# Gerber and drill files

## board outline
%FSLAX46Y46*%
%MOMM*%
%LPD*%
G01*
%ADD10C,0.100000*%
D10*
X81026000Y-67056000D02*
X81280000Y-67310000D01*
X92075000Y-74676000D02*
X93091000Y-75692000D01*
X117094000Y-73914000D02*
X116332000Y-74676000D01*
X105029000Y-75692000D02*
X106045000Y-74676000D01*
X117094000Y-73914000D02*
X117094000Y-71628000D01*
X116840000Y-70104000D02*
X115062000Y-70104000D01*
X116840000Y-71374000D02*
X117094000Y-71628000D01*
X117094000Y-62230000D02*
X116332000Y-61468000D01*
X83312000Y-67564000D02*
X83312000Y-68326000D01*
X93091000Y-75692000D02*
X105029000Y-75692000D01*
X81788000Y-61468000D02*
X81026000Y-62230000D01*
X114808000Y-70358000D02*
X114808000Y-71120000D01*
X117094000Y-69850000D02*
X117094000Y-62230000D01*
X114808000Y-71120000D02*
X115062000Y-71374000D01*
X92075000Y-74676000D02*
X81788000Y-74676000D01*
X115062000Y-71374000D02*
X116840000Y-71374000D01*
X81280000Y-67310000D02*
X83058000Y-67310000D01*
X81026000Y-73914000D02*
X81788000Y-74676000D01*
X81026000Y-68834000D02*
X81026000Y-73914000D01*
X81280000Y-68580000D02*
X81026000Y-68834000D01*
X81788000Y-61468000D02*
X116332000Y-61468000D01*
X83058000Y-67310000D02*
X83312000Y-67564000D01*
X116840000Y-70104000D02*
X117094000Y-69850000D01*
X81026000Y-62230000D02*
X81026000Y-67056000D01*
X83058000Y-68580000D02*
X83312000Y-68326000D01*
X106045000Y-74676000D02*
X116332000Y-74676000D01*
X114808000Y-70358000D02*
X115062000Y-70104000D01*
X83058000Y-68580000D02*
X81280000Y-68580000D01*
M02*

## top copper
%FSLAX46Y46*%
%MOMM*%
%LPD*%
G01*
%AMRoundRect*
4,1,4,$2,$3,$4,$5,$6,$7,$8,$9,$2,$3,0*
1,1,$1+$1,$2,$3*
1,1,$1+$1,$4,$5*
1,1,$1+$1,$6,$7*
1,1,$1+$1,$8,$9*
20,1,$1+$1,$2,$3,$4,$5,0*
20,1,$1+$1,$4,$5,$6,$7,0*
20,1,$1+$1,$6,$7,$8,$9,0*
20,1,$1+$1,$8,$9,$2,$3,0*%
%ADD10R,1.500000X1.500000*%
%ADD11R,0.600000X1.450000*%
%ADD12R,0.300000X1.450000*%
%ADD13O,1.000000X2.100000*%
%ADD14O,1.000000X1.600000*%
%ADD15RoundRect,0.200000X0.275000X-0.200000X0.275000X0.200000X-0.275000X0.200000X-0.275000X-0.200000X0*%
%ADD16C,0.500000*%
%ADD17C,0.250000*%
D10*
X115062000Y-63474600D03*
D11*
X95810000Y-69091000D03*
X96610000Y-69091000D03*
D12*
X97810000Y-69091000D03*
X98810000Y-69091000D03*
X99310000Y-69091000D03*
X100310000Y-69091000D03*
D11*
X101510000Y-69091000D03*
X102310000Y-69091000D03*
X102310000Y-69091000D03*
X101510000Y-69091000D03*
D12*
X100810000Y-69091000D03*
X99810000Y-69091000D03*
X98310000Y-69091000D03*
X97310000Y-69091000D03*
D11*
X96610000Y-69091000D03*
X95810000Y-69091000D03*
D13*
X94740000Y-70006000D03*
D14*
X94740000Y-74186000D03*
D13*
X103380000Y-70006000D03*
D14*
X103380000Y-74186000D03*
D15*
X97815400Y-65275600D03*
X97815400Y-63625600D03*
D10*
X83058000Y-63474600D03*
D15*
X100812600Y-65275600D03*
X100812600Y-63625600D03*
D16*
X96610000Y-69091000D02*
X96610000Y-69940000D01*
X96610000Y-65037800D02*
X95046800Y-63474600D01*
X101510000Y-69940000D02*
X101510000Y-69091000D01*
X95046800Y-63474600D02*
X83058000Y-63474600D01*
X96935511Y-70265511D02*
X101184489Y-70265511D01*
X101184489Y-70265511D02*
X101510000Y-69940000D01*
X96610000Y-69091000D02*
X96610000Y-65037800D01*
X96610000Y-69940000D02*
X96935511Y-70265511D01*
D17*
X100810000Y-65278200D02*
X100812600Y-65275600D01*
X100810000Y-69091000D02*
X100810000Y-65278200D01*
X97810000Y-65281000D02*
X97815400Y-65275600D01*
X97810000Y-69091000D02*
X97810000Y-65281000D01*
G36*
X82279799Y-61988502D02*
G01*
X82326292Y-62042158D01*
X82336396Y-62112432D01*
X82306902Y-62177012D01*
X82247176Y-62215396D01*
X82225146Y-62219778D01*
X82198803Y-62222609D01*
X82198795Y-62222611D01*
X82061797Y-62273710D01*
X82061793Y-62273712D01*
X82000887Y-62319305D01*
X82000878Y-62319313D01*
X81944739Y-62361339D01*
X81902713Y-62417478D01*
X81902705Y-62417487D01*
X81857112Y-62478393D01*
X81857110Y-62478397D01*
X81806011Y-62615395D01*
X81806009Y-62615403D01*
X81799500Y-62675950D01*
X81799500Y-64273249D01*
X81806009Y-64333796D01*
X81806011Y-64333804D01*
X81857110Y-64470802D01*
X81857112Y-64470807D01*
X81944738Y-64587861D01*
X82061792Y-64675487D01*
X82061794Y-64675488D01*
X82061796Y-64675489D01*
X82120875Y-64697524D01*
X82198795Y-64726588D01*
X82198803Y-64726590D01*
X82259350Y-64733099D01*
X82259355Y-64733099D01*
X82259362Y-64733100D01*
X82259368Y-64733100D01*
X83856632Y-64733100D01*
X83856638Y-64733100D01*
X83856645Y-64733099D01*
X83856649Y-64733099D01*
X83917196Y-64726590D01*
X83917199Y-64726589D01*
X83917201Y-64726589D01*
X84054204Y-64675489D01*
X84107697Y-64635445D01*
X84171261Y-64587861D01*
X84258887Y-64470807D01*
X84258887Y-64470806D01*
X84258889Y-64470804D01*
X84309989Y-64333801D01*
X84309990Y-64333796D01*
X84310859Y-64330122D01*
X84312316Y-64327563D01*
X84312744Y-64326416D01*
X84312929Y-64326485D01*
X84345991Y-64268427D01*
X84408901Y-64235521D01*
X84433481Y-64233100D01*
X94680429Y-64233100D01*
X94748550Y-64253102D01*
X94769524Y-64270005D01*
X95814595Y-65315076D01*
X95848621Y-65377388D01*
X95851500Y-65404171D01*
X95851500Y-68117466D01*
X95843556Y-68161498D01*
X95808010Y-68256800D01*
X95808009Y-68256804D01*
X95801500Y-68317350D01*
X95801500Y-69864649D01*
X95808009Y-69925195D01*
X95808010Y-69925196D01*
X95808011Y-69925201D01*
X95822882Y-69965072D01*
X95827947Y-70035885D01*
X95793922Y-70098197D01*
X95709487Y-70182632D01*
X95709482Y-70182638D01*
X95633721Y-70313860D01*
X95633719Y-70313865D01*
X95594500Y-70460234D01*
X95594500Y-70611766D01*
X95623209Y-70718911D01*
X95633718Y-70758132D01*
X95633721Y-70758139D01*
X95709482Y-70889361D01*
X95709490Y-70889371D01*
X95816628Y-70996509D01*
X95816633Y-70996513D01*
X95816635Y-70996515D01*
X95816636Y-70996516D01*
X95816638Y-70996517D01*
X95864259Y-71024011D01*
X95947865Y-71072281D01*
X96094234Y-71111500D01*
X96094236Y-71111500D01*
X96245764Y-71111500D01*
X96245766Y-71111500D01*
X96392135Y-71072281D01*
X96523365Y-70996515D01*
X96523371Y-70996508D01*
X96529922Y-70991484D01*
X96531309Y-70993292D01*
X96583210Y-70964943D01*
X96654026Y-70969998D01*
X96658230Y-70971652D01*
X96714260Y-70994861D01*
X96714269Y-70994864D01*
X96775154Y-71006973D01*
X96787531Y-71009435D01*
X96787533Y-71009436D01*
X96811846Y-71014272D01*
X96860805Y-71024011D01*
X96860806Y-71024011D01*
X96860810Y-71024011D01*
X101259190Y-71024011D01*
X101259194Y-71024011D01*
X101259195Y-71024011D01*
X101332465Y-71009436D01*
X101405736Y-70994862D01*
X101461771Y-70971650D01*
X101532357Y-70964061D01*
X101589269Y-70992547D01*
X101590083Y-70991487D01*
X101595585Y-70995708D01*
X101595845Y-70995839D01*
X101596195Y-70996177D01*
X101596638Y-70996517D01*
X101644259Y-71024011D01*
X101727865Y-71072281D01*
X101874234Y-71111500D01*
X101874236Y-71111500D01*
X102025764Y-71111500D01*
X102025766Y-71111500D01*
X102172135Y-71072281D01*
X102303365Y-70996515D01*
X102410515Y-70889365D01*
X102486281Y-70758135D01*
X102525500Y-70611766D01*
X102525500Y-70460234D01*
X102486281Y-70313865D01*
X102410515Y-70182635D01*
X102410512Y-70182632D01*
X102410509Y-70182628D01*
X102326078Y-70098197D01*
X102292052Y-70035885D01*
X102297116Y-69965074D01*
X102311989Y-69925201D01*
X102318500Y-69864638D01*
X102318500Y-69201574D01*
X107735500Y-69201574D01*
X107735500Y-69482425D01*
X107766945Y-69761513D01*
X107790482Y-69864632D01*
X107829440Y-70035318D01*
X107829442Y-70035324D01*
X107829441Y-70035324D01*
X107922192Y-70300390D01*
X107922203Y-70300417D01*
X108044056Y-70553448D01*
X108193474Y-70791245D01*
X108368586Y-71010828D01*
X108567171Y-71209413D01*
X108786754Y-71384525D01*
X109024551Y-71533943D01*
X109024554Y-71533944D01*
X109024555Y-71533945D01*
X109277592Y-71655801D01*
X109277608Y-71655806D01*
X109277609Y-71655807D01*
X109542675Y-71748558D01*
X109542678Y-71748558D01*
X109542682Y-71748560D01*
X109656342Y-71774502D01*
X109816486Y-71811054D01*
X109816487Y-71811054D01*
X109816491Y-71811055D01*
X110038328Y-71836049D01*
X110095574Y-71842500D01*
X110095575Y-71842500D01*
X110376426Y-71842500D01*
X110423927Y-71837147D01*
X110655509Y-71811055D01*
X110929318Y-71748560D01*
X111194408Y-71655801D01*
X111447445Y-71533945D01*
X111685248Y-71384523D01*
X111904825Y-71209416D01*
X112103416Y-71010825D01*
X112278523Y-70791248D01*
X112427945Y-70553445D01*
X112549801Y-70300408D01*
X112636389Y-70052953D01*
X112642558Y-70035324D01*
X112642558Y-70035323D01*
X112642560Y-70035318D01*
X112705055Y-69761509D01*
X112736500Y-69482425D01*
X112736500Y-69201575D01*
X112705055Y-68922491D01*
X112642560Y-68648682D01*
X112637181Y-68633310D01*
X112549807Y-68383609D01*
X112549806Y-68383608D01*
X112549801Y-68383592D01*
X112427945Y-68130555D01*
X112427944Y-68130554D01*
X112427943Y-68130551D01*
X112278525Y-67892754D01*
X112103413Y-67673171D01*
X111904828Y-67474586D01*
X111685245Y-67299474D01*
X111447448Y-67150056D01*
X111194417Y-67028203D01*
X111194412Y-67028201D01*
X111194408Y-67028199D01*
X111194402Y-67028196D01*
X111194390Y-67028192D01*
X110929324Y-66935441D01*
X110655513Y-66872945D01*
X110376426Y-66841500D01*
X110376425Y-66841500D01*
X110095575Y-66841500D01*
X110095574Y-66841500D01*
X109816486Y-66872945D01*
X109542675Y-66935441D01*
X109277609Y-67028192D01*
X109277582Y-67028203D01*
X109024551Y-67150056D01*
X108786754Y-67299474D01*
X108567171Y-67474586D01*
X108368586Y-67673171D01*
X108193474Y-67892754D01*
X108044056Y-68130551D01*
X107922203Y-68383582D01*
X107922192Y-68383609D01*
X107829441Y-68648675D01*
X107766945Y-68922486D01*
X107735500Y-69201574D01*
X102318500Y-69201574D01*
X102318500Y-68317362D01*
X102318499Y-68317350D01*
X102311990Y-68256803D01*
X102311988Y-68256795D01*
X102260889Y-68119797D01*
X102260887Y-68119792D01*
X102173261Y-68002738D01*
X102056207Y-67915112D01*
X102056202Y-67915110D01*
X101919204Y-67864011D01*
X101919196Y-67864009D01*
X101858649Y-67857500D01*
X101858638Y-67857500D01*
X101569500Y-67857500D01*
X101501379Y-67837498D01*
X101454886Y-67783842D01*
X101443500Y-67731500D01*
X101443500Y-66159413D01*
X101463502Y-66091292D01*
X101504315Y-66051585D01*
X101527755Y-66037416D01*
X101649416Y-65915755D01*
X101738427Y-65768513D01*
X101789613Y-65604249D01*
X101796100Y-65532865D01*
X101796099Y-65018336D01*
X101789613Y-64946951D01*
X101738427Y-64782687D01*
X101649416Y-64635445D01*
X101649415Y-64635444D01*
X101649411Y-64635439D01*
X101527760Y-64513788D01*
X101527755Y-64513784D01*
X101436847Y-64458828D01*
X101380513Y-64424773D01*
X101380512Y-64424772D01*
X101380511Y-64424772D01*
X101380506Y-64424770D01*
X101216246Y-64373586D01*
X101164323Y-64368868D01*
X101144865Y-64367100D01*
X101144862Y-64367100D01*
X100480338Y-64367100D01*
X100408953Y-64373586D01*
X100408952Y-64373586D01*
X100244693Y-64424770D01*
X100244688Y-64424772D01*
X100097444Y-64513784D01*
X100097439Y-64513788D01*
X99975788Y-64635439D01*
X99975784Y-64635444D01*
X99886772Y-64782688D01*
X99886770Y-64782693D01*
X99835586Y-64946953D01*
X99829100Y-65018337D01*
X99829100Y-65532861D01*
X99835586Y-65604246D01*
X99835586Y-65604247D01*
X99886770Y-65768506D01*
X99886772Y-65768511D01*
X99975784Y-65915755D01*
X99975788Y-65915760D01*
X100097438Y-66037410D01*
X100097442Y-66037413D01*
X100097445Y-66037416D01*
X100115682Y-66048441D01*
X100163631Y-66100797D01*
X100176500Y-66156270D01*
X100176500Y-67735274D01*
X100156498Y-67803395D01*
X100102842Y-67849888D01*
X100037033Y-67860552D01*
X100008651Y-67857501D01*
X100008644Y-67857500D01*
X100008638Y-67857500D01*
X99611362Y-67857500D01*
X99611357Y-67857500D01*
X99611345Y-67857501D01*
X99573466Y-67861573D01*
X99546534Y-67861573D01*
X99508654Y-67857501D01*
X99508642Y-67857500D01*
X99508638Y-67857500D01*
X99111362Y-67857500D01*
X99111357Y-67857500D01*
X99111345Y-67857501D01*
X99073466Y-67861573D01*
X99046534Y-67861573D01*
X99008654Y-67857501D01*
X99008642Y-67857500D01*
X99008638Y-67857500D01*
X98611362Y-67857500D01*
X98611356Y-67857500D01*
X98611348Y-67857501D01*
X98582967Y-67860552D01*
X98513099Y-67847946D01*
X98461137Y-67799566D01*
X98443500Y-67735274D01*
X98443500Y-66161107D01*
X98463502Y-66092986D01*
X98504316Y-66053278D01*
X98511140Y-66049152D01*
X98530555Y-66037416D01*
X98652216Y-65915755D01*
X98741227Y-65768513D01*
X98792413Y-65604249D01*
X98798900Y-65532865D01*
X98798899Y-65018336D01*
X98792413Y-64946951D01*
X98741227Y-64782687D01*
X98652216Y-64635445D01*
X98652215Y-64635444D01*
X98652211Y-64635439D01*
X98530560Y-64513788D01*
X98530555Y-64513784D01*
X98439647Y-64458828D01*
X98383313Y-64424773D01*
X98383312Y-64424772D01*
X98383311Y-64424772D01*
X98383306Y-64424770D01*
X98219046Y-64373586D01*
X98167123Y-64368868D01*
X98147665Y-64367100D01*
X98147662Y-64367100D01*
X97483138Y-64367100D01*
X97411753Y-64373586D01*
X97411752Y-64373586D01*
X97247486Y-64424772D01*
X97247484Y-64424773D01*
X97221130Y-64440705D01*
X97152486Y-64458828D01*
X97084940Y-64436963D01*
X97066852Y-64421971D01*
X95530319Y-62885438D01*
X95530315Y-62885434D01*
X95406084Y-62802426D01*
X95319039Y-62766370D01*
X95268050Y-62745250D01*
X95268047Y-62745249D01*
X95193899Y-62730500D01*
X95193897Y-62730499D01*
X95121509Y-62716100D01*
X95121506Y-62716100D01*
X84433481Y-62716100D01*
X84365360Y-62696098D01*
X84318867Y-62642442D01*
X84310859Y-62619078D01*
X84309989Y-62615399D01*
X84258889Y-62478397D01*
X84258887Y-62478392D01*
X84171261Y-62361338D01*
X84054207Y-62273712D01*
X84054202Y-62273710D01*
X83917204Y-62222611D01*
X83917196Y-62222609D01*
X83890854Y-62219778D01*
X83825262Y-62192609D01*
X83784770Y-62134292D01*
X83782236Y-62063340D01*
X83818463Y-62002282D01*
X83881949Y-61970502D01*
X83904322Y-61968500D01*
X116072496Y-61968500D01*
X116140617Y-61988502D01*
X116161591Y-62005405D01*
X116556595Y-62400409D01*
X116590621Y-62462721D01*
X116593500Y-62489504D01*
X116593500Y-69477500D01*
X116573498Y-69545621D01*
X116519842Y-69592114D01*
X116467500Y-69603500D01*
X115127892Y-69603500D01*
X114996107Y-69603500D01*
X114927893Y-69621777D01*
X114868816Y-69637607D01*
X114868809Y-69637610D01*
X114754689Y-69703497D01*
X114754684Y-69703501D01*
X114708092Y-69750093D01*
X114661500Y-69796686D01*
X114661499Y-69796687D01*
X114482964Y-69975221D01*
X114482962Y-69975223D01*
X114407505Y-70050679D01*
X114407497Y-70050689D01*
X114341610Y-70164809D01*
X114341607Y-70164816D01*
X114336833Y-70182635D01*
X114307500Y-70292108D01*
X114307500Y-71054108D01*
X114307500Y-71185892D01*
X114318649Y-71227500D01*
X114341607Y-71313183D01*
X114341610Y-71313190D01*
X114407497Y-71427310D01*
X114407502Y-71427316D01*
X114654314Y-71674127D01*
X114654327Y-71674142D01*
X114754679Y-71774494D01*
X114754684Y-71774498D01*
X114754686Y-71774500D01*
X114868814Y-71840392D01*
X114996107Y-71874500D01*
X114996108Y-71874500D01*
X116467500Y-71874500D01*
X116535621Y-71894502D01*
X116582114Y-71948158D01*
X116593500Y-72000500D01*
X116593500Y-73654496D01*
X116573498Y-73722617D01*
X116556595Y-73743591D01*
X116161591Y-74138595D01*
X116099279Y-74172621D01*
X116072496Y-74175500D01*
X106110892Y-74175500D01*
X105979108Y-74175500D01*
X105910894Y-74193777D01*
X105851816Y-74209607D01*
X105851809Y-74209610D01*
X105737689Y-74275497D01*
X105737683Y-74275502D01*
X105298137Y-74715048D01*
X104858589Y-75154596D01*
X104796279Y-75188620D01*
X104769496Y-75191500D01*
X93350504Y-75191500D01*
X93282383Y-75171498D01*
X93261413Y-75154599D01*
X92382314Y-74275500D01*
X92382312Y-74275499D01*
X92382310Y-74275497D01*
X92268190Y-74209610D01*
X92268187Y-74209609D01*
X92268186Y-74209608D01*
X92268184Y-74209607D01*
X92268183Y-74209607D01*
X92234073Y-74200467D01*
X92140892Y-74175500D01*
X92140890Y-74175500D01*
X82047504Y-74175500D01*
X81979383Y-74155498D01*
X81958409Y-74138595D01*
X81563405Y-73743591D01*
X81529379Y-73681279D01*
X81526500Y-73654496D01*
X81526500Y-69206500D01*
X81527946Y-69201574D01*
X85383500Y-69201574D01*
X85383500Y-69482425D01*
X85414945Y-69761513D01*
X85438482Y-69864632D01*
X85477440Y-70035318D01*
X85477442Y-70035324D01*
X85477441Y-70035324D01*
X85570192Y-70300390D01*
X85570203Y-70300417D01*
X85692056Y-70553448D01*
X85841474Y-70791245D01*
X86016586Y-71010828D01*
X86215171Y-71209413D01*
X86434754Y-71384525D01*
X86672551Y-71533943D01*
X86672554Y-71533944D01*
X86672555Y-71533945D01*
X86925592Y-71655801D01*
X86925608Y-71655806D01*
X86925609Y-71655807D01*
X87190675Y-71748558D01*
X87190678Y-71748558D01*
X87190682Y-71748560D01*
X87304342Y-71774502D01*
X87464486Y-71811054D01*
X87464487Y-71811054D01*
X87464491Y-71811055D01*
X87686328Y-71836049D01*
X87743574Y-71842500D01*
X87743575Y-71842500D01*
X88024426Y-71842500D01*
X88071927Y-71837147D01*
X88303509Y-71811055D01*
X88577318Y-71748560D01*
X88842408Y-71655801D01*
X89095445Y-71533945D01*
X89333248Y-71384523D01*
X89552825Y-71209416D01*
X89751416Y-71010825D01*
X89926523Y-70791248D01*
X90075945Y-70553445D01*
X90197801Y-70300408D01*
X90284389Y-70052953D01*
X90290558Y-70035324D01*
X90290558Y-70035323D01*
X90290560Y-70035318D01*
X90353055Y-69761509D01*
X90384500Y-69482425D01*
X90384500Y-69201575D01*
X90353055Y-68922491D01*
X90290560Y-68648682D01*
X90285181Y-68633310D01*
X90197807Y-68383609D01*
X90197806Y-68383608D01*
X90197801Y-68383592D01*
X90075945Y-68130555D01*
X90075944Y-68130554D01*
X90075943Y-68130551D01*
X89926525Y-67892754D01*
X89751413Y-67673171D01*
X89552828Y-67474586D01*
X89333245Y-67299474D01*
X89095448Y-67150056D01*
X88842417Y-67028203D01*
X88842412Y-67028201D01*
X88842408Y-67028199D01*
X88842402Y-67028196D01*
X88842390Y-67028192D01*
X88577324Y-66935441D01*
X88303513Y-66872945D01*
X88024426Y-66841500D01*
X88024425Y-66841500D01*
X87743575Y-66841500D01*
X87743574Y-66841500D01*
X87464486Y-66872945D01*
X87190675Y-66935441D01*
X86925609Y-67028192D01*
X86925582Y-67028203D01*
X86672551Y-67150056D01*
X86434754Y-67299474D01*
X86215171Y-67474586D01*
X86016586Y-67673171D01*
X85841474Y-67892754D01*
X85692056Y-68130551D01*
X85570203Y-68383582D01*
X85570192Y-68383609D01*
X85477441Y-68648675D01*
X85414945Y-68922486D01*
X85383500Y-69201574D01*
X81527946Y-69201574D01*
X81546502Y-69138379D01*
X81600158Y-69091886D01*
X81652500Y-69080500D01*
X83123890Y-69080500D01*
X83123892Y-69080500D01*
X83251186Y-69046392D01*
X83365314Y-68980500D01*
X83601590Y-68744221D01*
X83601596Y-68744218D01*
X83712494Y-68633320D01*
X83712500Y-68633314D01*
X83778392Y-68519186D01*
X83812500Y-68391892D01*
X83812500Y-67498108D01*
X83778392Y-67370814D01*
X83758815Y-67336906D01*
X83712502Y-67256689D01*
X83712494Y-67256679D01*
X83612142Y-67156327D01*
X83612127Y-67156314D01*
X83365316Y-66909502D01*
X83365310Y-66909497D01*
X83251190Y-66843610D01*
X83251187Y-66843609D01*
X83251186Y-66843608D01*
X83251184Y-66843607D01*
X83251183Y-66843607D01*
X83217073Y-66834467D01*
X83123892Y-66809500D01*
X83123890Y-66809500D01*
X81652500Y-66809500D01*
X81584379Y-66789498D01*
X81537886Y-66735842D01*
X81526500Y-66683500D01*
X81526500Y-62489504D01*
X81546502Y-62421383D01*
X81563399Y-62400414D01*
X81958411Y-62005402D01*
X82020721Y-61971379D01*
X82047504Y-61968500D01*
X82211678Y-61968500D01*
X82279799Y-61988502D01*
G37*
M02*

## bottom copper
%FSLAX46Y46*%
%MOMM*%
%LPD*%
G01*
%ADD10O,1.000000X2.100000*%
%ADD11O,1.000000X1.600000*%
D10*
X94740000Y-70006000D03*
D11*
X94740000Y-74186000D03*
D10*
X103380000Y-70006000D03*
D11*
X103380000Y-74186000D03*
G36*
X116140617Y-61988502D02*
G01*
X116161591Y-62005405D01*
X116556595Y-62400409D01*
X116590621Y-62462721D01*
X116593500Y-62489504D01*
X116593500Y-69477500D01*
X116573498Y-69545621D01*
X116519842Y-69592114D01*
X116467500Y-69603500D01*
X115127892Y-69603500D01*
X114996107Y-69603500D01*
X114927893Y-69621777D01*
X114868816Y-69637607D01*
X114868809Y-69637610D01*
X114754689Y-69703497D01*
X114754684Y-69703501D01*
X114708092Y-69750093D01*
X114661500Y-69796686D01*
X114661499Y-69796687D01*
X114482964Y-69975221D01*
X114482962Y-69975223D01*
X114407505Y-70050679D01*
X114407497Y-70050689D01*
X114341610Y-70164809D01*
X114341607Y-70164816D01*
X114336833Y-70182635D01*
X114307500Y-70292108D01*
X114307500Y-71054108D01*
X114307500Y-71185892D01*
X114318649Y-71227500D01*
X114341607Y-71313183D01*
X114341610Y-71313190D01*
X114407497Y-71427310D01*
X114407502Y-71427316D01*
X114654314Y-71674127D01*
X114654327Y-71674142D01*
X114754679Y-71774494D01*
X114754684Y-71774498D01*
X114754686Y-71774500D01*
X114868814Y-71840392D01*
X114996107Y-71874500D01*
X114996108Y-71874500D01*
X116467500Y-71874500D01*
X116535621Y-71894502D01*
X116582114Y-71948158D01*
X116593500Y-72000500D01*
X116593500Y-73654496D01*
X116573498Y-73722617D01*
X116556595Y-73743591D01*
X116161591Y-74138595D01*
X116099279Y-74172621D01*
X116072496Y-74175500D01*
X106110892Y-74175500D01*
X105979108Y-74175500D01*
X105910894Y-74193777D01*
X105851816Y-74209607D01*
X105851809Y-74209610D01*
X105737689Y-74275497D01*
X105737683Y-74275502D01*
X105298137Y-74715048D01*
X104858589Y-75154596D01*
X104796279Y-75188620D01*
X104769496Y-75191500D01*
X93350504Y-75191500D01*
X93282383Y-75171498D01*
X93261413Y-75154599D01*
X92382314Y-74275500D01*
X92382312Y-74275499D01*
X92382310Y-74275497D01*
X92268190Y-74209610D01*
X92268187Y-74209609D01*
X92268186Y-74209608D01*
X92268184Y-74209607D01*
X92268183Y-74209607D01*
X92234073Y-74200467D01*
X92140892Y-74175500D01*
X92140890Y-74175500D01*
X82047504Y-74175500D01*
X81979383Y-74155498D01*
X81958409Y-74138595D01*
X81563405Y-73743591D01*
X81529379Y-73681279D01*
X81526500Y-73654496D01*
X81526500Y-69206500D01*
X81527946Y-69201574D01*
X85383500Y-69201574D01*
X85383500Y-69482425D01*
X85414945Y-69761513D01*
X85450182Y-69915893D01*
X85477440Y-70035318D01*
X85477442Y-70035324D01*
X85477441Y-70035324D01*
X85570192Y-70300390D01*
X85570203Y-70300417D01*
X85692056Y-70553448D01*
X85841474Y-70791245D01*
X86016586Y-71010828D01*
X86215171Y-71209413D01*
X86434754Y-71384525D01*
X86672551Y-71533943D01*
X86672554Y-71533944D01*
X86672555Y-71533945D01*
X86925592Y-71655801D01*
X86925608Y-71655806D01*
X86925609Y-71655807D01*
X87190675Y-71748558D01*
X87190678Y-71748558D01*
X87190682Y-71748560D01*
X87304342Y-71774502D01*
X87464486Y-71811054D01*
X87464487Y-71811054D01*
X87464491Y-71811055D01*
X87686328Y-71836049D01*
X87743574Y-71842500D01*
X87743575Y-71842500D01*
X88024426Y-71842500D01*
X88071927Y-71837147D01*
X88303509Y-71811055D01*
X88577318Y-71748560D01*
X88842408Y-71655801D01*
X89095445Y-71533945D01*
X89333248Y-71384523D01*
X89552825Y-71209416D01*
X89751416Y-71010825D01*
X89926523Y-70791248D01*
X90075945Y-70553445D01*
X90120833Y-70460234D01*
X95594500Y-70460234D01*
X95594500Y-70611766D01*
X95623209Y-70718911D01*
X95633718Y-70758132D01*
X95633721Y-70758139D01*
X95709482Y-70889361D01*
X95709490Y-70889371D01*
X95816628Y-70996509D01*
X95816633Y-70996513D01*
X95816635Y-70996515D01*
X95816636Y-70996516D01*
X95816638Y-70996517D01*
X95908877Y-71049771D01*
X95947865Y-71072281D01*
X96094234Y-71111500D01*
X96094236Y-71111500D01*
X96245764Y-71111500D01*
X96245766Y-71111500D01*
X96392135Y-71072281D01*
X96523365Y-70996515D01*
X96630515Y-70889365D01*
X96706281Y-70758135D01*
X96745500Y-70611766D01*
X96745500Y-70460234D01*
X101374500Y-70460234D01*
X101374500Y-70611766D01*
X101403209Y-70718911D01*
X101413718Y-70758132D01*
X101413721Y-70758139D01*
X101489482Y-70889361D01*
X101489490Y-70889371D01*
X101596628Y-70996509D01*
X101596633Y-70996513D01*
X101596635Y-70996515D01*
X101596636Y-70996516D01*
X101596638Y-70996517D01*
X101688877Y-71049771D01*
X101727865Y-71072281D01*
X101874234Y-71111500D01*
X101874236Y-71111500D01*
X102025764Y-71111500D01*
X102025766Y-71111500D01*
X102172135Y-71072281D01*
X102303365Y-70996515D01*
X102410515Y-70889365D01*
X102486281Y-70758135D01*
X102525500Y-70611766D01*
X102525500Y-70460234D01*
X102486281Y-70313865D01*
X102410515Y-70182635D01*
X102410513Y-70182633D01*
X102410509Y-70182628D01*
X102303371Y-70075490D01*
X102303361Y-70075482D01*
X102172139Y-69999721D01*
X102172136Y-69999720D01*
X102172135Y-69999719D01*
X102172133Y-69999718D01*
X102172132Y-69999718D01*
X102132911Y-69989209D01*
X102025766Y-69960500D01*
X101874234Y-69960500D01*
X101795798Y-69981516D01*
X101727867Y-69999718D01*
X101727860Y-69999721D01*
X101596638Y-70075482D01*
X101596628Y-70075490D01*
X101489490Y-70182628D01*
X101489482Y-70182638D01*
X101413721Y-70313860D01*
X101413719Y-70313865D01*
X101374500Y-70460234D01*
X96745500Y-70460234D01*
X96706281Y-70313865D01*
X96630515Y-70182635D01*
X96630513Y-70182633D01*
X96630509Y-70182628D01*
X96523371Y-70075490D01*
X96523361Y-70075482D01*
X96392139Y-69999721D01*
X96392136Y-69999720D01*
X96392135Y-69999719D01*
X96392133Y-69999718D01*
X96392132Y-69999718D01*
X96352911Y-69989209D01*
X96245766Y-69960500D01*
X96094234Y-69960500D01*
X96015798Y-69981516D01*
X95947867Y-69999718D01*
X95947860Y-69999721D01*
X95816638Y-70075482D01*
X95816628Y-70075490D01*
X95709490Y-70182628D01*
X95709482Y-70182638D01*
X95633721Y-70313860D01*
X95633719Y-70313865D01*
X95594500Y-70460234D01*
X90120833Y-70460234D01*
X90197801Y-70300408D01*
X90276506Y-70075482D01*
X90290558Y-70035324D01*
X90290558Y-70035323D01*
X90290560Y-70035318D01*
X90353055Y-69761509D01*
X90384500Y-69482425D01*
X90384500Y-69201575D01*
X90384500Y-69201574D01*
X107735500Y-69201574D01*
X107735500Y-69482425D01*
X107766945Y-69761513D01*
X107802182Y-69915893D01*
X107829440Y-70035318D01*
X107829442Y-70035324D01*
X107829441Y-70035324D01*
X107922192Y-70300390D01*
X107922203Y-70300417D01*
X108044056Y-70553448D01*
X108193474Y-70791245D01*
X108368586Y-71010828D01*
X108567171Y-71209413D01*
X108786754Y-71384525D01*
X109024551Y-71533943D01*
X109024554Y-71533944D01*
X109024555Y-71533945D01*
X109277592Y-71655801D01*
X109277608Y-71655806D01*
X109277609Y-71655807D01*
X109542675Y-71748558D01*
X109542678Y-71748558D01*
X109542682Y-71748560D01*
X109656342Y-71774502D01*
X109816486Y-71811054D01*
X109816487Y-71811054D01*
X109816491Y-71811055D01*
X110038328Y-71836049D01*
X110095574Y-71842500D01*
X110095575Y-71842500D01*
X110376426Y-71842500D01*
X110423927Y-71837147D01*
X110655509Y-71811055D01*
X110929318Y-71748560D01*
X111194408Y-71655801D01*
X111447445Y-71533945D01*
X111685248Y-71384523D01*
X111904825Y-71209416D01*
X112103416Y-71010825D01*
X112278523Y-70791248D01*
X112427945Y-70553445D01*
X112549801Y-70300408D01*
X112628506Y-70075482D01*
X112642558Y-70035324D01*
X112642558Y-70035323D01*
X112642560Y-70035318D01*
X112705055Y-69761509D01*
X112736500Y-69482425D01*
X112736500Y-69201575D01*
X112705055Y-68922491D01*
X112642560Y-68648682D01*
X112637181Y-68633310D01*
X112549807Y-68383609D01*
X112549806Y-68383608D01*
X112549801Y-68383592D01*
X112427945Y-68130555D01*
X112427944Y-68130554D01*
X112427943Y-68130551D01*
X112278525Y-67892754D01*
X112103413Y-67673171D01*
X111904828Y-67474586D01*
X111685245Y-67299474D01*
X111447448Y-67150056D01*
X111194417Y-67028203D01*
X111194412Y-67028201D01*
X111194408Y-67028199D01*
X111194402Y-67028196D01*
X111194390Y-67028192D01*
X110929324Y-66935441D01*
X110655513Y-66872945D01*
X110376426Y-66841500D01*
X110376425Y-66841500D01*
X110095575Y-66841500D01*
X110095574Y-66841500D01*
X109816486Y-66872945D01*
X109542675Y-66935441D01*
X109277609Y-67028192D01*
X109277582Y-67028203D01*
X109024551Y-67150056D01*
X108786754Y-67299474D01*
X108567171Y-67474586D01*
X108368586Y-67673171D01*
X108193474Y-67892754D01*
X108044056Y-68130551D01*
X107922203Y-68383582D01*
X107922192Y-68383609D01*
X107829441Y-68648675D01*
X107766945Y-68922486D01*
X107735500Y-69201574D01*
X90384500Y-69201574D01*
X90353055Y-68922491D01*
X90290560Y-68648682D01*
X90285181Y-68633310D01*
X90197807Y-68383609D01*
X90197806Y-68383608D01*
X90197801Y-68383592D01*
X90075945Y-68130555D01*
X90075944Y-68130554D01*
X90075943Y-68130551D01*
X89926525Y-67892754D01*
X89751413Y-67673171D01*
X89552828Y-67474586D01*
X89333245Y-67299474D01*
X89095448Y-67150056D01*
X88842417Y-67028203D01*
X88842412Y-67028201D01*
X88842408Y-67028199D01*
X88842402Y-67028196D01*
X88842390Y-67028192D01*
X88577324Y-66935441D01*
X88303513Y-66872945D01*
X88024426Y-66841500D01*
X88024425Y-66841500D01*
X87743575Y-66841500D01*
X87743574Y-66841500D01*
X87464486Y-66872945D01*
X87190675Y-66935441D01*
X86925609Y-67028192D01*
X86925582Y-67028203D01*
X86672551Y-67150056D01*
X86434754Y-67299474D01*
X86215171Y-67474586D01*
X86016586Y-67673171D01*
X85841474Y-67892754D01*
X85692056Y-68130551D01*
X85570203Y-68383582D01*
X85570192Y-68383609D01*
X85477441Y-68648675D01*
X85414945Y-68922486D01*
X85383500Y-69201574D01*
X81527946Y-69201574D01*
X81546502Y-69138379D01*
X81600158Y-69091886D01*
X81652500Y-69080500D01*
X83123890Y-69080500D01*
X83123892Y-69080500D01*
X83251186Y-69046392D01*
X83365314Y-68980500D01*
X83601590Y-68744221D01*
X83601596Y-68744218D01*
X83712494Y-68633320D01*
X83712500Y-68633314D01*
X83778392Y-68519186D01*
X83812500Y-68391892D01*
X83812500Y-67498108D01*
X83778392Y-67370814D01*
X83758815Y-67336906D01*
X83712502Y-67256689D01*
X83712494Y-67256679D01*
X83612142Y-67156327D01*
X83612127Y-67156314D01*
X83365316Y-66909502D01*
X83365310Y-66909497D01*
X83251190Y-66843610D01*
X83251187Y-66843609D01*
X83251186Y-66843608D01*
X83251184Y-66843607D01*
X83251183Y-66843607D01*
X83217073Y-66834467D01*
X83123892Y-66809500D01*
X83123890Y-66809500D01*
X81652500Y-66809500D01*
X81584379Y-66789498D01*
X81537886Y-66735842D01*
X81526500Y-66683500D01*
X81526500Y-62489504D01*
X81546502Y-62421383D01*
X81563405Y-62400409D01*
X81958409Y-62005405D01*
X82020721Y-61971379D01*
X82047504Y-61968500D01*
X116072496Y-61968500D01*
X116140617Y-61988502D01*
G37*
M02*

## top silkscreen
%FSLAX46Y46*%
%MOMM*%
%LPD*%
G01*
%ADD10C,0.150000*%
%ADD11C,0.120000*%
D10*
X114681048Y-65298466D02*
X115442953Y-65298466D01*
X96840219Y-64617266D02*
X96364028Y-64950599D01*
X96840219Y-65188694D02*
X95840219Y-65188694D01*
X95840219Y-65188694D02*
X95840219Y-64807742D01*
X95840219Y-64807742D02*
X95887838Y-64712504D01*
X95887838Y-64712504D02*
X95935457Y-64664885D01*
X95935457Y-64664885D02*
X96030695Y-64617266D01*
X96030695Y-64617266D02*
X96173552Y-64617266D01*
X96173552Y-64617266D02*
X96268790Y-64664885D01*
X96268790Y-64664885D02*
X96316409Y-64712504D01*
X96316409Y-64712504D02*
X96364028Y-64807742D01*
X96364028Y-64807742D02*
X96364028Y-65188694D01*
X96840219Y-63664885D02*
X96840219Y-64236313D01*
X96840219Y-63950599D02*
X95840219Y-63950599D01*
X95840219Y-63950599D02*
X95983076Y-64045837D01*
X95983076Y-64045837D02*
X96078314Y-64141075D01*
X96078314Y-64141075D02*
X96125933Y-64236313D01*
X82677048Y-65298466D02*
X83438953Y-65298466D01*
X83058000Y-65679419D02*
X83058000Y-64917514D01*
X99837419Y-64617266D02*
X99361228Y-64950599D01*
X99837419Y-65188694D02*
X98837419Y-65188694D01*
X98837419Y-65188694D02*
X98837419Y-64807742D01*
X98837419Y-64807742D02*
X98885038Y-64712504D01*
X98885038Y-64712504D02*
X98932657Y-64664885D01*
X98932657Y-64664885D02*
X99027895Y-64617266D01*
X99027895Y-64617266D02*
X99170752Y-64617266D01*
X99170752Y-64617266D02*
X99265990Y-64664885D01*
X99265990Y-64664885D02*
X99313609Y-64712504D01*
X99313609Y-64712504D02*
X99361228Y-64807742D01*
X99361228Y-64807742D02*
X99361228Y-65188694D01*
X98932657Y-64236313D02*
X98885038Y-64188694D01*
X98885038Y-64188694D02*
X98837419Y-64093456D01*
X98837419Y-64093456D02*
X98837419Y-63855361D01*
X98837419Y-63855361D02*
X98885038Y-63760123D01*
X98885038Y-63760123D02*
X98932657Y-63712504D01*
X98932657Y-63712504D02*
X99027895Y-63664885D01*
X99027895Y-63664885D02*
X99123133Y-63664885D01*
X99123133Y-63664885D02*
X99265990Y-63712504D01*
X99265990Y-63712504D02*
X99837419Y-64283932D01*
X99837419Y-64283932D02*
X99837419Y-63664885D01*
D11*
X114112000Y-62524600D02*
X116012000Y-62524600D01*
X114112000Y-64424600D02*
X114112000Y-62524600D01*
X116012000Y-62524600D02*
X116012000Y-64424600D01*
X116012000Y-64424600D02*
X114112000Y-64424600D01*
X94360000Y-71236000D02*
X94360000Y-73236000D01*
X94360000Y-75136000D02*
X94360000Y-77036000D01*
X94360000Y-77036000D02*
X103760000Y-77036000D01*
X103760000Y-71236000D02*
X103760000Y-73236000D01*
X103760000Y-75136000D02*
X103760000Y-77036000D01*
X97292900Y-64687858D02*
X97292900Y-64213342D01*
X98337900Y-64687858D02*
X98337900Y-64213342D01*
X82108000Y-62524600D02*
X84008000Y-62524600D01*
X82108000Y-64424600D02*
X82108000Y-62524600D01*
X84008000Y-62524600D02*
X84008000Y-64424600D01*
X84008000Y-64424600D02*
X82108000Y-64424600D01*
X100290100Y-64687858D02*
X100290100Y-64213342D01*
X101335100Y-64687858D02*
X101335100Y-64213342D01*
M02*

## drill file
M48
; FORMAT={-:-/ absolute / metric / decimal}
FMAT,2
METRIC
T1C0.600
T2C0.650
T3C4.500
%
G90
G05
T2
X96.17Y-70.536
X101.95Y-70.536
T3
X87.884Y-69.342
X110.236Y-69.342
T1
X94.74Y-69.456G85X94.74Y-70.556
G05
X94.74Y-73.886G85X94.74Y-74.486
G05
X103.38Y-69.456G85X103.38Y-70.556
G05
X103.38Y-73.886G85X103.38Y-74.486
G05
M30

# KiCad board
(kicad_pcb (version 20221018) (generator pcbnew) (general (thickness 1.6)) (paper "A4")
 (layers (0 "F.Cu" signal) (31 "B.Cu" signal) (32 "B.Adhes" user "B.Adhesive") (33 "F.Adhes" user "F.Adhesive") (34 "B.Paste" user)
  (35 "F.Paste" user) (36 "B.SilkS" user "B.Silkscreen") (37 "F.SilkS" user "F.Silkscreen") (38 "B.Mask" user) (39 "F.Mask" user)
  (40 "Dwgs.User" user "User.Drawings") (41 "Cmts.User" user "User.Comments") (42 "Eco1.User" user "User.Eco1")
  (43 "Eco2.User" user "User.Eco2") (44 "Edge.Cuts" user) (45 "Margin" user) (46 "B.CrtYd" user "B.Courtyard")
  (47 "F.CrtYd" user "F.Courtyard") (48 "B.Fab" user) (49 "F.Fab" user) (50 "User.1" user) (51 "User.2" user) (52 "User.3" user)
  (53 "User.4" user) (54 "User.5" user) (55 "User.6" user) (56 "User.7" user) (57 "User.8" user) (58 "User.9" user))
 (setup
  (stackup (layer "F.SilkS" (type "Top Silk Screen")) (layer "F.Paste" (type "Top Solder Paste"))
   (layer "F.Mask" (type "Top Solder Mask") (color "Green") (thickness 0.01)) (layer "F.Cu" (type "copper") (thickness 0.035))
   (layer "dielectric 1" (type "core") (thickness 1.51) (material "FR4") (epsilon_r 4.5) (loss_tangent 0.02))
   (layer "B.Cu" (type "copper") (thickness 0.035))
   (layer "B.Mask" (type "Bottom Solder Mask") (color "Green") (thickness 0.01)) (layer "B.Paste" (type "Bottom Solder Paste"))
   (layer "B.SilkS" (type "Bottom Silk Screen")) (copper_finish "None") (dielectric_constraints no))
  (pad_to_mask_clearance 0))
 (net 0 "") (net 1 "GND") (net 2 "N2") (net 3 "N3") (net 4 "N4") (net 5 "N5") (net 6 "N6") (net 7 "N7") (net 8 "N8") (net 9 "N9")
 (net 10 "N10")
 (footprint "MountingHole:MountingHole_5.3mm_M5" (layer "F.Cu") (at 87.884 69.342)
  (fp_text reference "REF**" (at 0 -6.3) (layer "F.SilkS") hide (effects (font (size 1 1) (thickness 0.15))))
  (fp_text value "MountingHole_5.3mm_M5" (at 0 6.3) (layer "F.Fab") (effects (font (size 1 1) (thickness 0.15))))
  (pad "" np_thru_hole circle (at 0 0) (size 4.5 4.5) (drill 4.5) (layers "F&B.Cu" "*.Mask")))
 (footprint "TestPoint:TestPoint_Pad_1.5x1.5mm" (layer "F.Cu") (at 115.062 63.4746)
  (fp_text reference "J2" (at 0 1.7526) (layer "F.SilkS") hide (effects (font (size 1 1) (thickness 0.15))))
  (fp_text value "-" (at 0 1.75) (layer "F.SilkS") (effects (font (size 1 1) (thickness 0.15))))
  (fp_line (start -0.95 -0.95) (end 0.95 -0.95) (stroke (width 0.12) (type solid)) (layer "F.SilkS"))
  (fp_line (start -0.95 0.95) (end -0.95 -0.95) (stroke (width 0.12) (type solid)) (layer "F.SilkS"))
  (fp_line (start 0.95 -0.95) (end 0.95 0.95) (stroke (width 0.12) (type solid)) (layer "F.SilkS"))
  (fp_line (start 0.95 0.95) (end -0.95 0.95) (stroke (width 0.12) (type solid)) (layer "F.SilkS"))
  (pad "1" smd rect (at 0 0) (size 1.5 1.5) (layers "F.Cu" "F.Mask") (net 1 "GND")))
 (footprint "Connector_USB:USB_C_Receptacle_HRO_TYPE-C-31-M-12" (layer "F.Cu") (at 99.06 73.136)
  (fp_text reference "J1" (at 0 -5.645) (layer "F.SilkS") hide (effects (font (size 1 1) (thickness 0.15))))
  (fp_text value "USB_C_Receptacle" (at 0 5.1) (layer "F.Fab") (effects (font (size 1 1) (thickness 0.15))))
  (fp_line (start -4.7 -1.9) (end -4.7 0.1) (stroke (width 0.12) (type solid)) (layer "F.SilkS"))
  (fp_line (start -4.7 2) (end -4.7 3.9) (stroke (width 0.12) (type solid)) (layer "F.SilkS"))
  (fp_line (start -4.7 3.9) (end 4.7 3.9) (stroke (width 0.12) (type solid)) (layer "F.SilkS"))
  (fp_line (start 4.7 -1.9) (end 4.7 0.1) (stroke (width 0.12) (type solid)) (layer "F.SilkS"))
  (fp_line (start 4.7 2) (end 4.7 3.9) (stroke (width 0.12) (type solid)) (layer "F.SilkS"))
  (pad "" np_thru_hole circle (at -2.89 -2.6) (size 0.65 0.65) (drill 0.65) (layers "*.Cu" "*.Mask"))
  (pad "" np_thru_hole circle (at 2.89 -2.6) (size 0.65 0.65) (drill 0.65) (layers "*.Cu" "*.Mask"))
  (pad "A1" smd rect (at -3.25 -4.045) (size 0.6 1.45) (layers "F.Cu" "F.Paste" "F.Mask") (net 1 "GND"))
  (pad "A4" smd rect (at -2.45 -4.045) (size 0.6 1.45) (layers "F.Cu" "F.Paste" "F.Mask") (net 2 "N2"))
  (pad "A5" smd rect (at -1.25 -4.045) (size 0.3 1.45) (layers "F.Cu" "F.Paste" "F.Mask") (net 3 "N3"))
  (pad "A6" smd rect (at -0.25 -4.045) (size 0.3 1.45) (layers "F.Cu" "F.Paste" "F.Mask") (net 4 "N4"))
  (pad "A7" smd rect (at 0.25 -4.045) (size 0.3 1.45) (layers "F.Cu" "F.Paste" "F.Mask") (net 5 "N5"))
  (pad "A8" smd rect (at 1.25 -4.045) (size 0.3 1.45) (layers "F.Cu" "F.Paste" "F.Mask") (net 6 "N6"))
  (pad "A9" smd rect (at 2.45 -4.045) (size 0.6 1.45) (layers "F.Cu" "F.Paste" "F.Mask") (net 2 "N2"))
  (pad "A12" smd rect (at 3.25 -4.045) (size 0.6 1.45) (layers "F.Cu" "F.Paste" "F.Mask") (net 1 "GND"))
  (pad "B1" smd rect (at 3.25 -4.045) (size 0.6 1.45) (layers "F.Cu" "F.Paste" "F.Mask") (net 1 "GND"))
  (pad "B4" smd rect (at 2.45 -4.045) (size 0.6 1.45) (layers "F.Cu" "F.Paste" "F.Mask") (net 2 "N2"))
  (pad "B5" smd rect (at 1.75 -4.045) (size 0.3 1.45) (layers "F.Cu" "F.Paste" "F.Mask") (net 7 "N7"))
  (pad "B6" smd rect (at 0.75 -4.045) (size 0.3 1.45) (layers "F.Cu" "F.Paste" "F.Mask") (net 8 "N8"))
  (pad "B7" smd rect (at -0.75 -4.045) (size 0.3 1.45) (layers "F.Cu" "F.Paste" "F.Mask") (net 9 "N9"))
  (pad "B8" smd rect (at -1.75 -4.045) (size 0.3 1.45) (layers "F.Cu" "F.Paste" "F.Mask") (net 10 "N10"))
  (pad "B9" smd rect (at -2.45 -4.045) (size 0.6 1.45) (layers "F.Cu" "F.Paste" "F.Mask") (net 2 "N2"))
  (pad "B12" smd rect (at -3.25 -4.045) (size 0.6 1.45) (layers "F.Cu" "F.Paste" "F.Mask") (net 1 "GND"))
  (pad "S1" thru_hole oval (at -4.32 -3.13) (size 1 2.1) (drill oval 0.6 1.7) (layers "*.Cu" "*.Mask") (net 1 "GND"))
  (pad "S1" thru_hole oval (at -4.32 1.05) (size 1 1.6) (drill oval 0.6 1.2) (layers "*.Cu" "*.Mask") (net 1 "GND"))
  (pad "S1" thru_hole oval (at 4.32 -3.13) (size 1 2.1) (drill oval 0.6 1.7) (layers "*.Cu" "*.Mask") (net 1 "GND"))
  (pad "S1" thru_hole oval (at 4.32 1.05) (size 1 1.6) (drill oval 0.6 1.2) (layers "*.Cu" "*.Mask") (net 1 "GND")))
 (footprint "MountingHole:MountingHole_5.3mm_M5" (layer "F.Cu") (at 110.236 69.342)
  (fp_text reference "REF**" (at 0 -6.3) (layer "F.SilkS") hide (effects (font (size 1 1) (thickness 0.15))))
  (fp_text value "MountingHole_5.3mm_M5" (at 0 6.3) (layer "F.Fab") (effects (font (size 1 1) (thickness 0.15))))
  (pad "" np_thru_hole circle (at 0 0) (size 4.5 4.5) (drill 4.5) (layers "F&B.Cu" "*.Mask")))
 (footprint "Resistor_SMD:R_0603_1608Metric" (layer "F.Cu") (at 97.8154 64.4506 90)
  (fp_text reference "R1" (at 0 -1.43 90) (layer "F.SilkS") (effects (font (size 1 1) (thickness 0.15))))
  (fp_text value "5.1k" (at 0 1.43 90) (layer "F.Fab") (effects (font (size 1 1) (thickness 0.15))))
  (fp_line (start -0.237258 -0.5225) (end 0.237258 -0.5225) (stroke (width 0.12) (type solid)) (layer "F.SilkS"))
  (fp_line (start -0.237258 0.5225) (end 0.237258 0.5225) (stroke (width 0.12) (type solid)) (layer "F.SilkS"))
  (pad "1" smd roundrect (at -0.825 0 90) (size 0.8 0.95) (layers "F.Cu" "F.Paste" "F.Mask") (roundrect_rratio 0.25) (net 3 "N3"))
  (pad "2" smd roundrect (at 0.825 0 90) (size 0.8 0.95) (layers "F.Cu" "F.Paste" "F.Mask") (roundrect_rratio 0.25) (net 1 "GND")))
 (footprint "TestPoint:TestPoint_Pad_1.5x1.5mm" (layer "F.Cu") (at 83.058 63.4746)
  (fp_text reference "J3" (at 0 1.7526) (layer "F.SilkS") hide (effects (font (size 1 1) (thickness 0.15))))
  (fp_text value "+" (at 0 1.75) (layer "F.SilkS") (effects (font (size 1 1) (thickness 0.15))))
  (fp_line (start -0.95 -0.95) (end 0.95 -0.95) (stroke (width 0.12) (type solid)) (layer "F.SilkS"))
  (fp_line (start -0.95 0.95) (end -0.95 -0.95) (stroke (width 0.12) (type solid)) (layer "F.SilkS"))
  (fp_line (start 0.95 -0.95) (end 0.95 0.95) (stroke (width 0.12) (type solid)) (layer "F.SilkS"))
  (fp_line (start 0.95 0.95) (end -0.95 0.95) (stroke (width 0.12) (type solid)) (layer "F.SilkS"))
  (pad "1" smd rect (at 0 0) (size 1.5 1.5) (layers "F.Cu" "F.Mask") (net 2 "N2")))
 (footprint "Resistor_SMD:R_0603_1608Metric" (layer "F.Cu") (at 100.8126 64.4506 90)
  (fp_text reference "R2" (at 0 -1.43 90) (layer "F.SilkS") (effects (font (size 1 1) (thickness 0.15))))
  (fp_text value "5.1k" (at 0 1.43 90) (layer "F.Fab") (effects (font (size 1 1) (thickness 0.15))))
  (fp_line (start -0.237258 -0.5225) (end 0.237258 -0.5225) (stroke (width 0.12) (type solid)) (layer "F.SilkS"))
  (fp_line (start -0.237258 0.5225) (end 0.237258 0.5225) (stroke (width 0.12) (type solid)) (layer "F.SilkS"))
  (pad "1" smd roundrect (at -0.825 0 90) (size 0.8 0.95) (layers "F.Cu" "F.Paste" "F.Mask") (roundrect_rratio 0.25) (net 7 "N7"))
  (pad "2" smd roundrect (at 0.825 0 90) (size 0.8 0.95) (layers "F.Cu" "F.Paste" "F.Mask") (roundrect_rratio 0.25) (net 1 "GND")))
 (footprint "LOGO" (layer "B.Cu") (at 111.0488 63.4492 180)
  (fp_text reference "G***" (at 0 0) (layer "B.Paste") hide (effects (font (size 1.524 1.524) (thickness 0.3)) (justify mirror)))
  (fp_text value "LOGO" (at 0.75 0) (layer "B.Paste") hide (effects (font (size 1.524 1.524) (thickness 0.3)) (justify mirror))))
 (gr_line (start 81.026 67.056) (end 81.28 67.31) (stroke (width 0.1) (type solid)) (layer "Edge.Cuts"))
 (gr_line (start 92.075 74.676) (end 93.091 75.692) (stroke (width 0.1) (type solid)) (layer "Edge.Cuts"))
 (gr_line (start 117.094 73.914) (end 116.332 74.676) (stroke (width 0.1) (type solid)) (layer "Edge.Cuts"))
 (gr_line (start 105.029 75.692) (end 106.045 74.676) (stroke (width 0.1) (type solid)) (layer "Edge.Cuts"))
 (gr_line (start 117.094 73.914) (end 117.094 71.628) (stroke (width 0.1) (type solid)) (layer "Edge.Cuts"))
 (gr_line (start 116.84 70.104) (end 115.062 70.104) (stroke (width 0.1) (type solid)) (layer "Edge.Cuts"))
 (gr_line (start 116.84 71.374) (end 117.094 71.628) (stroke (width 0.1) (type solid)) (layer "Edge.Cuts"))
 (gr_line (start 117.094 62.23) (end 116.332 61.468) (stroke (width 0.1) (type solid)) (layer "Edge.Cuts"))
 (gr_line (start 83.312 67.564) (end 83.312 68.326) (stroke (width 0.1) (type solid)) (layer "Edge.Cuts"))
 (gr_line (start 93.091 75.692) (end 105.029 75.692) (stroke (width 0.1) (type solid)) (layer "Edge.Cuts"))
 (gr_line (start 81.788 61.468) (end 81.026 62.23) (stroke (width 0.1) (type solid)) (layer "Edge.Cuts"))
 (gr_line (start 114.808 70.358) (end 114.808 71.12) (stroke (width 0.1) (type solid)) (layer "Edge.Cuts"))
 (gr_line (start 117.094 69.85) (end 117.094 62.23) (stroke (width 0.1) (type solid)) (layer "Edge.Cuts"))
 (gr_line (start 114.808 71.12) (end 115.062 71.374) (stroke (width 0.1) (type solid)) (layer "Edge.Cuts"))
 (gr_line (start 92.075 74.676) (end 81.788 74.676) (stroke (width 0.1) (type solid)) (layer "Edge.Cuts"))
 (gr_line (start 115.062 71.374) (end 116.84 71.374) (stroke (width 0.1) (type solid)) (layer "Edge.Cuts"))
 (gr_line (start 81.28 67.31) (end 83.058 67.31) (stroke (width 0.1) (type solid)) (layer "Edge.Cuts"))
 (gr_line (start 81.026 73.914) (end 81.788 74.676) (stroke (width 0.1) (type solid)) (layer "Edge.Cuts"))
 (gr_line (start 81.026 68.834) (end 81.026 73.914) (stroke (width 0.1) (type solid)) (layer "Edge.Cuts"))
 (gr_line (start 81.28 68.58) (end 81.026 68.834) (stroke (width 0.1) (type solid)) (layer "Edge.Cuts"))
 (gr_line (start 81.788 61.468) (end 116.332 61.468) (stroke (width 0.1) (type solid)) (layer "Edge.Cuts"))
 (gr_line (start 83.058 67.31) (end 83.312 67.564) (stroke (width 0.1) (type solid)) (layer "Edge.Cuts"))
 (gr_line (start 116.84 70.104) (end 117.094 69.85) (stroke (width 0.1) (type solid)) (layer "Edge.Cuts"))
 (gr_line (start 81.026 62.23) (end 81.026 67.056) (stroke (width 0.1) (type solid)) (layer "Edge.Cuts"))
 (gr_line (start 83.058 68.58) (end 83.312 68.326) (stroke (width 0.1) (type solid)) (layer "Edge.Cuts"))
 (gr_line (start 106.045 74.676) (end 116.332 74.676) (stroke (width 0.1) (type solid)) (layer "Edge.Cuts"))
 (gr_line (start 114.808 70.358) (end 115.062 70.104) (stroke (width 0.1) (type solid)) (layer "Edge.Cuts"))
 (gr_line (start 83.058 68.58) (end 81.28 68.58) (stroke (width 0.1) (type solid)) (layer "Edge.Cuts"))
 (segment (start 96.61 69.091) (end 96.61 69.94) (width 0.5) (layer "F.Cu") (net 2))
 (segment (start 96.61 65.0378) (end 95.0468 63.4746) (width 0.5) (layer "F.Cu") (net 2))
 (segment (start 101.51 69.94) (end 101.51 69.091) (width 0.5) (layer "F.Cu") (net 2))
 (segment (start 95.0468 63.4746) (end 83.058 63.4746) (width 0.5) (layer "F.Cu") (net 2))
 (segment (start 96.935511 70.265511) (end 101.184489 70.265511) (width 0.5) (layer "F.Cu") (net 2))
 (segment (start 101.184489 70.265511) (end 101.51 69.94) (width 0.5) (layer "F.Cu") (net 2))
 (segment (start 96.61 69.091) (end 96.61 65.0378) (width 0.5) (layer "F.Cu") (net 2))
 (segment (start 96.61 69.94) (end 96.935511 70.265511) (width 0.5) (layer "F.Cu") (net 2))
 (segment (start 100.81 65.2782) (end 100.8126 65.2756) (width 0.25) (layer "F.Cu") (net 7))
 (segment (start 100.81 69.091) (end 100.81 65.2782) (width 0.25) (layer "F.Cu") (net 7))
 (segment (start 97.81 65.281) (end 97.8154 65.2756) (width 0.25) (layer "F.Cu") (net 3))
 (segment (start 97.81 69.091) (end 97.81 65.281) (width 0.25) (layer "F.Cu") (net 3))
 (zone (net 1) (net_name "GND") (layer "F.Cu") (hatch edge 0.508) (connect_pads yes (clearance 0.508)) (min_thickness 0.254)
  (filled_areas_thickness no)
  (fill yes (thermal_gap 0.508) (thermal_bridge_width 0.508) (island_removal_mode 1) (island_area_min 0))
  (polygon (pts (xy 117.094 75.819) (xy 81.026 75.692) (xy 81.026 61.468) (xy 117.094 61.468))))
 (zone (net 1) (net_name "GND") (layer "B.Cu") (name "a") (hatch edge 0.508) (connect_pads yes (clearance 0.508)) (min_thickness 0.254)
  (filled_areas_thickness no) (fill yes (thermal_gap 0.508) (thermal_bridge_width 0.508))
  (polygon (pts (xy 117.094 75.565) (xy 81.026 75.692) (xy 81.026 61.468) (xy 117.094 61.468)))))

